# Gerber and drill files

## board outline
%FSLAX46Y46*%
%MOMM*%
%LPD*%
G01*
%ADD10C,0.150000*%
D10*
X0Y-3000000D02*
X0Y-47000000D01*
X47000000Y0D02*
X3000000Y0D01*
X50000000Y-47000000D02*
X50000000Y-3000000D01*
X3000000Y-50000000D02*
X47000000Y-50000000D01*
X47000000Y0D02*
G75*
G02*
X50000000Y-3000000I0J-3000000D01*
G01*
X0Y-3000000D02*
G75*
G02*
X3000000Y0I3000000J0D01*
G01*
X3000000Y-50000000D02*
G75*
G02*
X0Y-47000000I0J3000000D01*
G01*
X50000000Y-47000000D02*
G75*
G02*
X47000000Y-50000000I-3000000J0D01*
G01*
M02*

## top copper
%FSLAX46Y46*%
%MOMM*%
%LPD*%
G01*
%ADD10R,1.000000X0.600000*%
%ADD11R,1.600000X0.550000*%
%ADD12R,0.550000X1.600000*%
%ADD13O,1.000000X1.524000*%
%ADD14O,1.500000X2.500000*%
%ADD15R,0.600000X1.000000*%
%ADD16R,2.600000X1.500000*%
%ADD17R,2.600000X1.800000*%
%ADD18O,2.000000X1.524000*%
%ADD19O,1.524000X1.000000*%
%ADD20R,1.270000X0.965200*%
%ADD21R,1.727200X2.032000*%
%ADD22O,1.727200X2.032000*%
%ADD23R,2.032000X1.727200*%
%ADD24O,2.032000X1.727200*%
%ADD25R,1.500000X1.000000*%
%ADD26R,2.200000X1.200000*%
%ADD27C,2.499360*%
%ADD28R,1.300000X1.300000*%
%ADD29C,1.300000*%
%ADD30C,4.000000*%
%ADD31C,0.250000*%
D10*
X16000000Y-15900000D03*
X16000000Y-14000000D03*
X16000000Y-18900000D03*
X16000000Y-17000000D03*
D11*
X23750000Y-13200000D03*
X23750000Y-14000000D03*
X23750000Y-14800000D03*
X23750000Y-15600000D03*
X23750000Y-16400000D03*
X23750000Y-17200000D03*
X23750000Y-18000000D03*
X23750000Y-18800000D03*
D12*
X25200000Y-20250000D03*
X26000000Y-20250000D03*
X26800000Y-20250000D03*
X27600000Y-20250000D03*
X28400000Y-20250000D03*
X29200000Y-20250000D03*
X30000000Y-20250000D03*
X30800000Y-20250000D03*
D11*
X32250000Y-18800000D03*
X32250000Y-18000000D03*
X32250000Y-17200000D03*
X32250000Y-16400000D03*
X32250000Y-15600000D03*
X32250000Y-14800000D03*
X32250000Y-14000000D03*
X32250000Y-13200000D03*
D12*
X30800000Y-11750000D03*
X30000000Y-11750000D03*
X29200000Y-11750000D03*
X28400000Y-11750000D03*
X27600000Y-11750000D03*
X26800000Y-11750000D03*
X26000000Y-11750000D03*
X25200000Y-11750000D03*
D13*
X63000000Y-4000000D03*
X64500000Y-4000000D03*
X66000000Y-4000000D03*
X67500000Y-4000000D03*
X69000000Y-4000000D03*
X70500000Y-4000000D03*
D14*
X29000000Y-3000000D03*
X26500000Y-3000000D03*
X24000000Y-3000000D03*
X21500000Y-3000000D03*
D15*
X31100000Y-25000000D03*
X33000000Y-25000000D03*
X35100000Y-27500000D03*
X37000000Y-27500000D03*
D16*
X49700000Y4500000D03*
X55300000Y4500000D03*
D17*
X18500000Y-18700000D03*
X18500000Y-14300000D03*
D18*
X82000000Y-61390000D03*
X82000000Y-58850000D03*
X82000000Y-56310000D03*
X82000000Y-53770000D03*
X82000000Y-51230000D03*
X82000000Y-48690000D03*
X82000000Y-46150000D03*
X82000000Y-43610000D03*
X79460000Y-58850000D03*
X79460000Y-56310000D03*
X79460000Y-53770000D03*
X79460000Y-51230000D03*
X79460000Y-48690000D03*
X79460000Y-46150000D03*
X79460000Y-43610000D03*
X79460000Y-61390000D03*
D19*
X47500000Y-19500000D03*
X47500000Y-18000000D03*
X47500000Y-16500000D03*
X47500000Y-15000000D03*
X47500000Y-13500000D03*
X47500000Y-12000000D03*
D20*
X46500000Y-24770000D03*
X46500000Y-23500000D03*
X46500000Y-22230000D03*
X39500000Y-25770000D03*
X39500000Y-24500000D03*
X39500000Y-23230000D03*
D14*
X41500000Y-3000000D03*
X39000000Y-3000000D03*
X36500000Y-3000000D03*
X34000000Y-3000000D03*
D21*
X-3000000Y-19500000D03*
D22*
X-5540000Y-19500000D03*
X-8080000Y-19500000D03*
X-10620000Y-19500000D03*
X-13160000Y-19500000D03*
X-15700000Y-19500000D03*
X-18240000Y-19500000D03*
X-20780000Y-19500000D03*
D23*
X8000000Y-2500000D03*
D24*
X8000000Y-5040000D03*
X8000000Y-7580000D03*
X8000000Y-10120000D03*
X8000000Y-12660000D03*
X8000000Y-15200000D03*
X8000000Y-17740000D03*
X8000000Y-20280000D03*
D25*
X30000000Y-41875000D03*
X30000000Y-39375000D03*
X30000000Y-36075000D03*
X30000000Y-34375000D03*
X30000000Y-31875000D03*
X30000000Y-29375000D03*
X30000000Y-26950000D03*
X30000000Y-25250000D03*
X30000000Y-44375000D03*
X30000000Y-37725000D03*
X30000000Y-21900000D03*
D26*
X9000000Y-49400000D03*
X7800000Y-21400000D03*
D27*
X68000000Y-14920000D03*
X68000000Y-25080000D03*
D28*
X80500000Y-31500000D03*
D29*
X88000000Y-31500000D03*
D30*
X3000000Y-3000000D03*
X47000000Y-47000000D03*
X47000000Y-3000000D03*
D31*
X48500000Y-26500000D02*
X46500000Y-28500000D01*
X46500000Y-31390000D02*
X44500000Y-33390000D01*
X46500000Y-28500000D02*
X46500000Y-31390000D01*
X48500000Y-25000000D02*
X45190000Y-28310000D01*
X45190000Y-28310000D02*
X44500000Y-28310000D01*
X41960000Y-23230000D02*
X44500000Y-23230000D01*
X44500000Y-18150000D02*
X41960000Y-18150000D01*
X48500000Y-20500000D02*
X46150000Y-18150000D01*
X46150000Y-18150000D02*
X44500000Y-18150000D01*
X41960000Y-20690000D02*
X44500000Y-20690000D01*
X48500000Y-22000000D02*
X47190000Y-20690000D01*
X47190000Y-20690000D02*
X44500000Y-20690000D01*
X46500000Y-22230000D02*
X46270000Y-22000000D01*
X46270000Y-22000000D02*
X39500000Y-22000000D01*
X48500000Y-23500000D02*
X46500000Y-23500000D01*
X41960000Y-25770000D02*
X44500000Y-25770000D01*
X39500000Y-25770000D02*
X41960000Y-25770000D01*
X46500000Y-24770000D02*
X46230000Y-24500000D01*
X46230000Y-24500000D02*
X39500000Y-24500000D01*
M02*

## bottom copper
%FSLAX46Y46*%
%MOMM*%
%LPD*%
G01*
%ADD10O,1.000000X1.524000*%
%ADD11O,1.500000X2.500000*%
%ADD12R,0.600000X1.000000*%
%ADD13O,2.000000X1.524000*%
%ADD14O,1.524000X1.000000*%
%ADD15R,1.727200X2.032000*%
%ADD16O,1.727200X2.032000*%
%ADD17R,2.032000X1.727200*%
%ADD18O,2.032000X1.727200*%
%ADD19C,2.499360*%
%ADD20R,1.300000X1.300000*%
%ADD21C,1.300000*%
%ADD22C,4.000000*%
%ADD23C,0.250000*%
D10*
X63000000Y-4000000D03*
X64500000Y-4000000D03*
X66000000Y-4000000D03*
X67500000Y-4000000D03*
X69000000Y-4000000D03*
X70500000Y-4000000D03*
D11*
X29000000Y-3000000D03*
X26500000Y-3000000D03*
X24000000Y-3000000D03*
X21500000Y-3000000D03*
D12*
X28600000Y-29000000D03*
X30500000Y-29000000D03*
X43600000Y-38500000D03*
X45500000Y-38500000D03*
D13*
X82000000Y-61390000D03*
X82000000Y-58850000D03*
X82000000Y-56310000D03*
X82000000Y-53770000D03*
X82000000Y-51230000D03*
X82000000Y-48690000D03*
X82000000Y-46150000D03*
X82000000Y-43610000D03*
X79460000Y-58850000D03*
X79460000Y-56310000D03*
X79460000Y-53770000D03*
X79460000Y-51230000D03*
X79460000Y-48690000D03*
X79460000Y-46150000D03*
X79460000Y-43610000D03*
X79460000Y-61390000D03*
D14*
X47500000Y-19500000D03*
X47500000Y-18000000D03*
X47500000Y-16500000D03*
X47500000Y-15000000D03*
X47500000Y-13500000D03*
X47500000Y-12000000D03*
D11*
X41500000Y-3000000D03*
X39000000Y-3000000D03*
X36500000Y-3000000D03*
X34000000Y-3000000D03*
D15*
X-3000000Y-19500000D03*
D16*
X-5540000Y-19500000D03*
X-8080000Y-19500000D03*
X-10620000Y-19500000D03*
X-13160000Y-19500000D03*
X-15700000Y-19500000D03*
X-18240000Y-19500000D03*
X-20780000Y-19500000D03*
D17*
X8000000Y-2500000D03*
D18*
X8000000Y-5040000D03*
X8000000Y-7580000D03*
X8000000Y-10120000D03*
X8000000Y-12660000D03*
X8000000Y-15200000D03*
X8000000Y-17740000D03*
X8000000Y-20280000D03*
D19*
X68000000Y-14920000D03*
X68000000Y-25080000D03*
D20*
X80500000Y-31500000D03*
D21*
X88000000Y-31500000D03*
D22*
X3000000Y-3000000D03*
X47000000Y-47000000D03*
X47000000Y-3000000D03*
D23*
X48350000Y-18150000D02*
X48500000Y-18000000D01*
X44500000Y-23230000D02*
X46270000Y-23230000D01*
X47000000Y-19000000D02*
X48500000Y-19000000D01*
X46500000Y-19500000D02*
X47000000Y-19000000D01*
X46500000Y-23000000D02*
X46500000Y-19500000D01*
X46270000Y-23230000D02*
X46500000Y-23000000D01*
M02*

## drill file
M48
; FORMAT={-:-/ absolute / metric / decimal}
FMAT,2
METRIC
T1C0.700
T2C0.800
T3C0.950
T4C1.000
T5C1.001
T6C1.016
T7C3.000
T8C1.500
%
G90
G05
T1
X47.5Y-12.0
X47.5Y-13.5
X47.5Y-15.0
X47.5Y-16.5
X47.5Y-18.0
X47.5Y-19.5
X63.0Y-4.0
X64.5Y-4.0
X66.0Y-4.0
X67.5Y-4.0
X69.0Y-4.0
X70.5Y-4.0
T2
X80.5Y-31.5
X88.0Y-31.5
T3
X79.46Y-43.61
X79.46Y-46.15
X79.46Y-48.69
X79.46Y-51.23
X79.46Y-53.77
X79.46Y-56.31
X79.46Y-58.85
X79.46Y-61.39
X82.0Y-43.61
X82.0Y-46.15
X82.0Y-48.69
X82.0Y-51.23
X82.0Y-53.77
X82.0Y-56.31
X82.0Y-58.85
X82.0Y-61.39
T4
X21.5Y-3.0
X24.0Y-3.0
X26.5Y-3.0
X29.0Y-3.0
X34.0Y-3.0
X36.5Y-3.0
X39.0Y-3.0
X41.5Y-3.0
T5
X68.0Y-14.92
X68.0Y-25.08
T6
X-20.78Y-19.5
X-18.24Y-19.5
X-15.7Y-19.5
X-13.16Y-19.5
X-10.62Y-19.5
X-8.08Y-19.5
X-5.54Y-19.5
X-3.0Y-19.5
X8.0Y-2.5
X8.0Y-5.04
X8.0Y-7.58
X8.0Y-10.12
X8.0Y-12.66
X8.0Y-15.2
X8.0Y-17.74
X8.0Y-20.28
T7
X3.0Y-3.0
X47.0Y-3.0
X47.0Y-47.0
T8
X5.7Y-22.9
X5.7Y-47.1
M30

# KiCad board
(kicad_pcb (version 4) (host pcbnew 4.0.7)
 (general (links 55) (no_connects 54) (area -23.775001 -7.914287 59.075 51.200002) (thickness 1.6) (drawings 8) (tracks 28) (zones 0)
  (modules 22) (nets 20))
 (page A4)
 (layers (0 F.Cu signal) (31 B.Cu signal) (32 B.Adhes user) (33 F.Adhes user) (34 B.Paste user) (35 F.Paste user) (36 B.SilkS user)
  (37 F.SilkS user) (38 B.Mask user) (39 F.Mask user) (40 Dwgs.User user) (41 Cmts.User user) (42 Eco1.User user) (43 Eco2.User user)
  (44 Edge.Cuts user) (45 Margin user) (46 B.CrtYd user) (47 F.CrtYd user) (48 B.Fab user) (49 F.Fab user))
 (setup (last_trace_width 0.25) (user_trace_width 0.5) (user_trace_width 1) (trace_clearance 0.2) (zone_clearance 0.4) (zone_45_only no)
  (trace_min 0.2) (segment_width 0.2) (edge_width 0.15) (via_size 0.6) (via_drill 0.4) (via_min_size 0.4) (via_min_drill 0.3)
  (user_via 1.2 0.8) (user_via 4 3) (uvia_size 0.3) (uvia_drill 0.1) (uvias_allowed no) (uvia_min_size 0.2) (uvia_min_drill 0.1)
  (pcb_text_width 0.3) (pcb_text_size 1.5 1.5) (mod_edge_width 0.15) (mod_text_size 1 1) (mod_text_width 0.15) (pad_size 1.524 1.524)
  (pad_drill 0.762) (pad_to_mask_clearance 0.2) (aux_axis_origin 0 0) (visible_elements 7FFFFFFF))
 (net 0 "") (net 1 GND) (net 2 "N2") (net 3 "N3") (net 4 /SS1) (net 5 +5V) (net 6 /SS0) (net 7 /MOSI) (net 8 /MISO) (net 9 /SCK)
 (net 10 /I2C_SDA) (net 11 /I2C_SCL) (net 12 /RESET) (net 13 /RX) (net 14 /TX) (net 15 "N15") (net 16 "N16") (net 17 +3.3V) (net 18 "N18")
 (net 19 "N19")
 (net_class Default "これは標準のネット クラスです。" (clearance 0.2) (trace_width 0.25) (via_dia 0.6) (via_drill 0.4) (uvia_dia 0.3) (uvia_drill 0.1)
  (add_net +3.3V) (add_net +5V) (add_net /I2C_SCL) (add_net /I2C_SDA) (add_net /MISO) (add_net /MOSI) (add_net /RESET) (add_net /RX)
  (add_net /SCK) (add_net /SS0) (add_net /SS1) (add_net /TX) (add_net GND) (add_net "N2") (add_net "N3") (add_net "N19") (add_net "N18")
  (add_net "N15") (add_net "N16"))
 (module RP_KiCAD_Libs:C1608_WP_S (layer F.Cu) (at 16 15 90)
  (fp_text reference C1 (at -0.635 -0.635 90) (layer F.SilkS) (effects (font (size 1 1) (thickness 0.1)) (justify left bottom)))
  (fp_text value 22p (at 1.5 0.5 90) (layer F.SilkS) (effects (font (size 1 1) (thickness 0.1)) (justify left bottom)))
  (pad 1 smd rect (at -0.9 0 90) (size 0.6 1) (layers F.Cu F.Paste F.Mask) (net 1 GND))
  (pad 2 smd rect (at 1 0 90) (size 0.6 1) (layers F.Cu F.Paste F.Mask) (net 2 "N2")))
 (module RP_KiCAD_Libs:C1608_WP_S (layer F.Cu) (at 16 18 90)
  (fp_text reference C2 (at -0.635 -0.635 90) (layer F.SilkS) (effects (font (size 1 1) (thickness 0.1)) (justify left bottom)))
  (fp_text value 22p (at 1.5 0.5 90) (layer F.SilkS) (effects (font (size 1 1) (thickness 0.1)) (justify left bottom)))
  (pad 1 smd rect (at -0.9 0 90) (size 0.6 1) (layers F.Cu F.Paste F.Mask) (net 1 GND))
  (pad 2 smd rect (at 1 0 90) (size 0.6 1) (layers F.Cu F.Paste F.Mask) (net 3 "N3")))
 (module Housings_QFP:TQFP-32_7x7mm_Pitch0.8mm (layer F.Cu) (at 28 16)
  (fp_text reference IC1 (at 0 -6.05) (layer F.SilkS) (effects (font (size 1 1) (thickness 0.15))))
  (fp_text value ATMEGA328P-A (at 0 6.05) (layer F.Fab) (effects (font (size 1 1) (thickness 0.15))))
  (pad 1 smd rect (at -4.25 -2.8) (size 1.6 0.55) (layers F.Cu F.Paste F.Mask))
  (pad 2 smd rect (at -4.25 -2) (size 1.6 0.55) (layers F.Cu F.Paste F.Mask) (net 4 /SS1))
  (pad 3 smd rect (at -4.25 -1.2) (size 1.6 0.55) (layers F.Cu F.Paste F.Mask) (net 1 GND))
  (pad 4 smd rect (at -4.25 -0.4) (size 1.6 0.55) (layers F.Cu F.Paste F.Mask) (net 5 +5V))
  (pad 5 smd rect (at -4.25 0.4) (size 1.6 0.55) (layers F.Cu F.Paste F.Mask) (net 1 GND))
  (pad 6 smd rect (at -4.25 1.2) (size 1.6 0.55) (layers F.Cu F.Paste F.Mask) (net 5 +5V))
  (pad 7 smd rect (at -4.25 2) (size 1.6 0.55) (layers F.Cu F.Paste F.Mask) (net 2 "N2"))
  (pad 8 smd rect (at -4.25 2.8) (size 1.6 0.55) (layers F.Cu F.Paste F.Mask) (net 3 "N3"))
  (pad 9 smd rect (at -2.8 4.25 90) (size 1.6 0.55) (layers F.Cu F.Paste F.Mask))
  (pad 10 smd rect (at -2 4.25 90) (size 1.6 0.55) (layers F.Cu F.Paste F.Mask))
  (pad 11 smd rect (at -1.2 4.25 90) (size 1.6 0.55) (layers F.Cu F.Paste F.Mask))
  (pad 12 smd rect (at -0.4 4.25 90) (size 1.6 0.55) (layers F.Cu F.Paste F.Mask))
  (pad 13 smd rect (at 0.4 4.25 90) (size 1.6 0.55) (layers F.Cu F.Paste F.Mask))
  (pad 14 smd rect (at 1.2 4.25 90) (size 1.6 0.55) (layers F.Cu F.Paste F.Mask) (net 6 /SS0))
  (pad 15 smd rect (at 2 4.25 90) (size 1.6 0.55) (layers F.Cu F.Paste F.Mask) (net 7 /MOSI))
  (pad 16 smd rect (at 2.8 4.25 90) (size 1.6 0.55) (layers F.Cu F.Paste F.Mask) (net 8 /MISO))
  (pad 17 smd rect (at 4.25 2.8) (size 1.6 0.55) (layers F.Cu F.Paste F.Mask) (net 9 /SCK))
  (pad 18 smd rect (at 4.25 2) (size 1.6 0.55) (layers F.Cu F.Paste F.Mask) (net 5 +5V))
  (pad 19 smd rect (at 4.25 1.2) (size 1.6 0.55) (layers F.Cu F.Paste F.Mask))
  (pad 20 smd rect (at 4.25 0.4) (size 1.6 0.55) (layers F.Cu F.Paste F.Mask) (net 5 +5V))
  (pad 21 smd rect (at 4.25 -0.4) (size 1.6 0.55) (layers F.Cu F.Paste F.Mask) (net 1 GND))
  (pad 22 smd rect (at 4.25 -1.2) (size 1.6 0.55) (layers F.Cu F.Paste F.Mask))
  (pad 23 smd rect (at 4.25 -2) (size 1.6 0.55) (layers F.Cu F.Paste F.Mask))
  (pad 24 smd rect (at 4.25 -2.8) (size 1.6 0.55) (layers F.Cu F.Paste F.Mask))
  (pad 25 smd rect (at 2.8 -4.25 90) (size 1.6 0.55) (layers F.Cu F.Paste F.Mask))
  (pad 26 smd rect (at 2 -4.25 90) (size 1.6 0.55) (layers F.Cu F.Paste F.Mask))
  (pad 27 smd rect (at 1.2 -4.25 90) (size 1.6 0.55) (layers F.Cu F.Paste F.Mask) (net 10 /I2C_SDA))
  (pad 28 smd rect (at 0.4 -4.25 90) (size 1.6 0.55) (layers F.Cu F.Paste F.Mask) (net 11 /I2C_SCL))
  (pad 29 smd rect (at -0.4 -4.25 90) (size 1.6 0.55) (layers F.Cu F.Paste F.Mask) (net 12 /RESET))
  (pad 30 smd rect (at -1.2 -4.25 90) (size 1.6 0.55) (layers F.Cu F.Paste F.Mask) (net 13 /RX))
  (pad 31 smd rect (at -2 -4.25 90) (size 1.6 0.55) (layers F.Cu F.Paste F.Mask) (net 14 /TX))
  (pad 32 smd rect (at -2.8 -4.25 90) (size 1.6 0.55) (layers F.Cu F.Paste F.Mask)))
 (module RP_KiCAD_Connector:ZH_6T (layer F.Cu) (at 63 4)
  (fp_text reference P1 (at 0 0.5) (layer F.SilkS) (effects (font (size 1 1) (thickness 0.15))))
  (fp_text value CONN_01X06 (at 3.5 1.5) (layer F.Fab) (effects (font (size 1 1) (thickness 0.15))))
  (pad 1 thru_hole oval (at 0 0) (size 1 1.524) (drill 0.7) (layers *.Cu *.Mask) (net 1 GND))
  (pad 2 thru_hole oval (at 1.5 0) (size 1 1.524) (drill 0.7) (layers *.Cu *.Mask) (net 5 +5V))
  (pad 3 thru_hole oval (at 3 0) (size 1 1.524) (drill 0.7) (layers *.Cu *.Mask) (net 12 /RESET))
  (pad 4 thru_hole oval (at 4.5 0) (size 1 1.524) (drill 0.7) (layers *.Cu *.Mask))
  (pad 5 thru_hole oval (at 6 0) (size 1 1.524) (drill 0.7) (layers *.Cu *.Mask) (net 14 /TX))
  (pad 6 thru_hole oval (at 7.5 0) (size 1 1.524) (drill 0.7) (layers *.Cu *.Mask) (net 13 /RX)))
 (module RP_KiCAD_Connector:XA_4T (layer F.Cu) (at 29 3 180)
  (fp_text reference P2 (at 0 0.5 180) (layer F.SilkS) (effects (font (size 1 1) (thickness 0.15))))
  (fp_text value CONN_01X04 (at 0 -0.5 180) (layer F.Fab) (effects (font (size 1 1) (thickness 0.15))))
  (pad 4 thru_hole oval (at 0 0 180) (size 1.5 2.5) (drill 1) (layers *.Cu *.Mask F.SilkS) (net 14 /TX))
  (pad 3 thru_hole oval (at 2.5 0 180) (size 1.5 2.5) (drill 1) (layers *.Cu *.Mask F.SilkS) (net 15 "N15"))
  (pad 2 thru_hole oval (at 5 0 180) (size 1.5 2.5) (drill 1) (layers *.Cu *.Mask F.SilkS) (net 5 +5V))
  (pad 1 thru_hole oval (at 7.5 0 180) (size 1.5 2.5) (drill 1) (layers *.Cu *.Mask F.SilkS) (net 1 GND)))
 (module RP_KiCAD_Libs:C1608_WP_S (layer B.Cu) (at 29.5 29)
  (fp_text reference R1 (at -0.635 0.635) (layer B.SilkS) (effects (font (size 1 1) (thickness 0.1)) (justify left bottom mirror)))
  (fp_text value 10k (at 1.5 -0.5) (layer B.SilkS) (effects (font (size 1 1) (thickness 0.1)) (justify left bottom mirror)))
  (pad 1 smd rect (at -0.9 0) (size 0.6 1) (layers B.Cu B.Paste B.Mask))
  (pad 2 smd rect (at 1 0) (size 0.6 1) (layers B.Cu B.Paste B.Mask) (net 12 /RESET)))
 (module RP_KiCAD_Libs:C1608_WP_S (layer B.Cu) (at 44.5 38.5)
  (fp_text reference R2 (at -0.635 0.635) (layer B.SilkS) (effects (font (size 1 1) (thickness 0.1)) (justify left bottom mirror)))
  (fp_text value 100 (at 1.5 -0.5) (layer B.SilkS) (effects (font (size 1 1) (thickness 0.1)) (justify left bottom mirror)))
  (pad 1 smd rect (at -0.9 0) (size 0.6 1) (layers B.Cu B.Paste B.Mask) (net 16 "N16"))
  (pad 2 smd rect (at 1 0) (size 0.6 1) (layers B.Cu B.Paste B.Mask) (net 12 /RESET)))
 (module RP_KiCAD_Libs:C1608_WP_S (layer F.Cu) (at 32 25)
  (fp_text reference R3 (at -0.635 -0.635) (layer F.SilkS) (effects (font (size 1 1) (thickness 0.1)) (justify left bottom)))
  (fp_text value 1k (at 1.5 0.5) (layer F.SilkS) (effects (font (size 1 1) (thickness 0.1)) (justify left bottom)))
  (pad 1 smd rect (at -0.9 0) (size 0.6 1) (layers F.Cu F.Paste F.Mask) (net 14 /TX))
  (pad 2 smd rect (at 1 0) (size 0.6 1) (layers F.Cu F.Paste F.Mask)))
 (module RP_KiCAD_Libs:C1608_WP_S (layer F.Cu) (at 36 27.5)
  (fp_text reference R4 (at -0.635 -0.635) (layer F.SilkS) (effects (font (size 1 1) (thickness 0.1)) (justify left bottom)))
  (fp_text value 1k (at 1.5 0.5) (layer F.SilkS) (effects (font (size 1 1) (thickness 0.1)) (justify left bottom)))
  (pad 1 smd rect (at -0.9 0) (size 0.6 1) (layers F.Cu F.Paste F.Mask) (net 13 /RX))
  (pad 2 smd rect (at 1 0) (size 0.6 1) (layers F.Cu F.Paste F.Mask) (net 15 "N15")))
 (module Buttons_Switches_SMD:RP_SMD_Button (layer F.Cu) (at 52.5 -4.5 180)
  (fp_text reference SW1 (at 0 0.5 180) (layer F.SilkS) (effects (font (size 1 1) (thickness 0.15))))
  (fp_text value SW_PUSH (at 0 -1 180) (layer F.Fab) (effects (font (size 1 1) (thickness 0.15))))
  (pad 1 smd rect (at 2.8 0 180) (size 2.6 1.5) (layers F.Cu F.Paste F.Mask) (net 16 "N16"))
  (pad 2 smd rect (at -2.8 0 180) (size 2.6 1.5) (layers F.Cu F.Paste F.Mask) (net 1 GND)))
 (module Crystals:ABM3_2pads (layer F.Cu) (at 18.5 16.5 90)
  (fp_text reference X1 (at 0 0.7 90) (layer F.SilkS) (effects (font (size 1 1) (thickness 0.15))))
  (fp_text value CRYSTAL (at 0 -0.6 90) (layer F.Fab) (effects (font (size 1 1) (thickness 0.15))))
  (pad 1 smd rect (at -2.2 0 90) (size 1.8 2.6) (layers F.Cu F.Paste F.Mask) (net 3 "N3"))
  (pad 2 smd rect (at 2.2 0 90) (size 1.8 2.6) (layers F.Cu F.Paste F.Mask) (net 2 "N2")))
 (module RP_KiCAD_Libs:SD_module (layer B.Cu) (at 82 52.5)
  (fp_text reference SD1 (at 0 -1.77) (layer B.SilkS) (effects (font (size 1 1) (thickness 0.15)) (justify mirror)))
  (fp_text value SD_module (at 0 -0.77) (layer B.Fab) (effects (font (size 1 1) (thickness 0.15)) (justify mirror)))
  (pad 1 thru_hole oval (at 0 8.89) (size 2 1.524) (drill 0.95) (layers *.Cu *.Mask) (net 1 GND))
  (pad 2 thru_hole oval (at 0 6.35) (size 2 1.524) (drill 0.95) (layers *.Cu *.Mask) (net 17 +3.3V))
  (pad 3 thru_hole oval (at 0 3.81) (size 2 1.524) (drill 0.95) (layers *.Cu *.Mask) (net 5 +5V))
  (pad 4 thru_hole oval (at 0 1.27) (size 2 1.524) (drill 0.95) (layers *.Cu *.Mask) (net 6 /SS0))
  (pad 5 thru_hole oval (at 0 -1.27) (size 2 1.524) (drill 0.95) (layers *.Cu *.Mask) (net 7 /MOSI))
  (pad 6 thru_hole oval (at 0 -3.81) (size 2 1.524) (drill 0.95) (layers *.Cu *.Mask) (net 9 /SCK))
  (pad 7 thru_hole oval (at 0 -6.35) (size 2 1.524) (drill 0.95) (layers *.Cu *.Mask) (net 8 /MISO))
  (pad 8 thru_hole oval (at 0 -8.89) (size 2 1.524) (drill 0.95) (layers *.Cu *.Mask) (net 1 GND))
  (pad 2 thru_hole oval (at -2.54 6.35) (size 2 1.524) (drill 0.95) (layers *.Cu *.Mask) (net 17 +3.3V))
  (pad 3 thru_hole oval (at -2.54 3.81) (size 2 1.524) (drill 0.95) (layers *.Cu *.Mask) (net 5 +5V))
  (pad 4 thru_hole oval (at -2.54 1.27) (size 2 1.524) (drill 0.95) (layers *.Cu *.Mask) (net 6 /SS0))
  (pad 5 thru_hole oval (at -2.54 -1.27) (size 2 1.524) (drill 0.95) (layers *.Cu *.Mask) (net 7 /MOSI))
  (pad 6 thru_hole oval (at -2.54 -3.81) (size 2 1.524) (drill 0.95) (layers *.Cu *.Mask) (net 9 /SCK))
  (pad 7 thru_hole oval (at -2.54 -6.35) (size 2 1.524) (drill 0.95) (layers *.Cu *.Mask) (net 8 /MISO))
  (pad 8 thru_hole oval (at -2.54 -8.89) (size 2 1.524) (drill 0.95) (layers *.Cu *.Mask) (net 1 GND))
  (pad 1 thru_hole oval (at -2.54 8.89) (size 2 1.524) (drill 0.95) (layers *.Cu *.Mask) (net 1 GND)))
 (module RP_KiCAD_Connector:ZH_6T (layer F.Cu) (at 47.5 19.5 90)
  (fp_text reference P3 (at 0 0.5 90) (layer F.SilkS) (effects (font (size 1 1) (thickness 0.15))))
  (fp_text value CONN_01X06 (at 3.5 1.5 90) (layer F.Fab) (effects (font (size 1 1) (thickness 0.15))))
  (pad 1 thru_hole oval (at 0 0 90) (size 1 1.524) (drill 0.7) (layers *.Cu *.Mask) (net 1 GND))
  (pad 2 thru_hole oval (at 1.5 0 90) (size 1 1.524) (drill 0.7) (layers *.Cu *.Mask) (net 5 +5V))
  (pad 3 thru_hole oval (at 3 0 90) (size 1 1.524) (drill 0.7) (layers *.Cu *.Mask) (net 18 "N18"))
  (pad 4 thru_hole oval (at 4.5 0 90) (size 1 1.524) (drill 0.7) (layers *.Cu *.Mask) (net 9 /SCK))
  (pad 5 thru_hole oval (at 6 0 90) (size 1 1.524) (drill 0.7) (layers *.Cu *.Mask) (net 8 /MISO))
  (pad 6 thru_hole oval (at 7.5 0 90) (size 1 1.524) (drill 0.7) (layers *.Cu *.Mask) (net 7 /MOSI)))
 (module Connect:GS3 (layer F.Cu) (at 46.5 23.5 180)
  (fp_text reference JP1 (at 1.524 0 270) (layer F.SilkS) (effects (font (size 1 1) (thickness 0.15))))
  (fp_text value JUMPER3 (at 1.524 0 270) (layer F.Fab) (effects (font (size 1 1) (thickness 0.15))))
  (pad 1 smd rect (at 0 -1.27 180) (size 1.27 0.9652) (layers F.Cu F.Paste F.Mask) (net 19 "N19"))
  (pad 2 smd rect (at 0 0 180) (size 1.27 0.9652) (layers F.Cu F.Paste F.Mask) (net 18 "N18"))
  (pad 3 smd rect (at 0 1.27 180) (size 1.27 0.9652) (layers F.Cu F.Paste F.Mask) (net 12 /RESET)))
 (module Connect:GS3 (layer F.Cu) (at 39.5 24.5 180)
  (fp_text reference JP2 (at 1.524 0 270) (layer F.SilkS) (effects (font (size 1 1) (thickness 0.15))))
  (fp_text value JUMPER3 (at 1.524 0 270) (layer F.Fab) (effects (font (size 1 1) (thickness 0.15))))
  (pad 1 smd rect (at 0 -1.27 180) (size 1.27 0.9652) (layers F.Cu F.Paste F.Mask) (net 6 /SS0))
  (pad 2 smd rect (at 0 0 180) (size 1.27 0.9652) (layers F.Cu F.Paste F.Mask) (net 19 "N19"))
  (pad 3 smd rect (at 0 1.27 180) (size 1.27 0.9652) (layers F.Cu F.Paste F.Mask) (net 4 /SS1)))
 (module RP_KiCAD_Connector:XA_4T (layer F.Cu) (at 41.5 3 180)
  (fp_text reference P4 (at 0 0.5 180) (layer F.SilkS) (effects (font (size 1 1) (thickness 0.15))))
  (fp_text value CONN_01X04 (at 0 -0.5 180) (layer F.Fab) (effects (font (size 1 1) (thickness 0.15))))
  (pad 4 thru_hole oval (at 0 0 180) (size 1.5 2.5) (drill 1) (layers *.Cu *.Mask F.SilkS) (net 10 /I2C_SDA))
  (pad 3 thru_hole oval (at 2.5 0 180) (size 1.5 2.5) (drill 1) (layers *.Cu *.Mask F.SilkS) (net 11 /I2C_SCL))
  (pad 2 thru_hole oval (at 5 0 180) (size 1.5 2.5) (drill 1) (layers *.Cu *.Mask F.SilkS) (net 5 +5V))
  (pad 1 thru_hole oval (at 7.5 0 180) (size 1.5 2.5) (drill 1) (layers *.Cu *.Mask F.SilkS) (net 1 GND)))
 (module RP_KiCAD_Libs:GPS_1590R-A (layer F.Cu) (at -38.5 -13)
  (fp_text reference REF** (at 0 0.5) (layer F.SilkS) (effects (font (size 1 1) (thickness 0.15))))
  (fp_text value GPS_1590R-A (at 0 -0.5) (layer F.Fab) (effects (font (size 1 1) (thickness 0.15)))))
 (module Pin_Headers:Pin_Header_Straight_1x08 (layer F.Cu) (at -3 19.5 270)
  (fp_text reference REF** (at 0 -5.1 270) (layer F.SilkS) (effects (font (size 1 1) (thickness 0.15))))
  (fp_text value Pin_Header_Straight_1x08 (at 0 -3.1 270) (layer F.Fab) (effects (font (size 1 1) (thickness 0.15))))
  (pad 1 thru_hole rect (at 0 0 270) (size 2.032 1.7272) (drill 1.016) (layers *.Cu *.Mask F.SilkS))
  (pad 2 thru_hole oval (at 0 2.54 270) (size 2.032 1.7272) (drill 1.016) (layers *.Cu *.Mask F.SilkS))
  (pad 3 thru_hole oval (at 0 5.08 270) (size 2.032 1.7272) (drill 1.016) (layers *.Cu *.Mask F.SilkS))
  (pad 4 thru_hole oval (at 0 7.62 270) (size 2.032 1.7272) (drill 1.016) (layers *.Cu *.Mask F.SilkS))
  (pad 5 thru_hole oval (at 0 10.16 270) (size 2.032 1.7272) (drill 1.016) (layers *.Cu *.Mask F.SilkS))
  (pad 6 thru_hole oval (at 0 12.7 270) (size 2.032 1.7272) (drill 1.016) (layers *.Cu *.Mask F.SilkS))
  (pad 7 thru_hole oval (at 0 15.24 270) (size 2.032 1.7272) (drill 1.016) (layers *.Cu *.Mask F.SilkS))
  (pad 8 thru_hole oval (at 0 17.78 270) (size 2.032 1.7272) (drill 1.016) (layers *.Cu *.Mask F.SilkS)))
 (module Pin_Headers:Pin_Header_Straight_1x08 (layer F.Cu) (at 8 2.5)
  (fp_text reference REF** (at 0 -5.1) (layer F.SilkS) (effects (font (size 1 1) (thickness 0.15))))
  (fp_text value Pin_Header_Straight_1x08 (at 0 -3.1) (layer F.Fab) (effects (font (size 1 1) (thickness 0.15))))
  (pad 1 thru_hole rect (at 0 0) (size 2.032 1.7272) (drill 1.016) (layers *.Cu *.Mask F.SilkS))
  (pad 2 thru_hole oval (at 0 2.54) (size 2.032 1.7272) (drill 1.016) (layers *.Cu *.Mask F.SilkS))
  (pad 3 thru_hole oval (at 0 5.08) (size 2.032 1.7272) (drill 1.016) (layers *.Cu *.Mask F.SilkS))
  (pad 4 thru_hole oval (at 0 7.62) (size 2.032 1.7272) (drill 1.016) (layers *.Cu *.Mask F.SilkS))
  (pad 5 thru_hole oval (at 0 10.16) (size 2.032 1.7272) (drill 1.016) (layers *.Cu *.Mask F.SilkS))
  (pad 6 thru_hole oval (at 0 12.7) (size 2.032 1.7272) (drill 1.016) (layers *.Cu *.Mask F.SilkS))
  (pad 7 thru_hole oval (at 0 15.24) (size 2.032 1.7272) (drill 1.016) (layers *.Cu *.Mask F.SilkS))
  (pad 8 thru_hole oval (at 0 17.78) (size 2.032 1.7272) (drill 1.016) (layers *.Cu *.Mask F.SilkS)))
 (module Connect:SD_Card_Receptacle (layer F.Cu) (at 30 35 270)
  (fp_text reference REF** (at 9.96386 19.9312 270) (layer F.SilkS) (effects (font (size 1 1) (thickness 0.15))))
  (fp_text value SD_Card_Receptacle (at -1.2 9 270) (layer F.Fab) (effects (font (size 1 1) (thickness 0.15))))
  (pad 1 smd rect (at 6.875 0 270) (size 1 1.5) (layers F.Cu F.Paste F.Mask))
  (pad 2 smd rect (at 4.375 0 270) (size 1 1.5) (layers F.Cu F.Paste F.Mask))
  (pad 3 smd rect (at 1.075 0 270) (size 1 1.5) (layers F.Cu F.Paste F.Mask))
  (pad 4 smd rect (at -0.625 0 270) (size 1 1.5) (layers F.Cu F.Paste F.Mask))
  (pad 5 smd rect (at -3.125 0 270) (size 1 1.5) (layers F.Cu F.Paste F.Mask))
  (pad 6 smd rect (at -5.625 0 270) (size 1 1.5) (layers F.Cu F.Paste F.Mask))
  (pad 7 smd rect (at -8.05 0 270) (size 1 1.5) (layers F.Cu F.Paste F.Mask))
  (pad 8 smd rect (at -9.75 0 270) (size 1 1.5) (layers F.Cu F.Paste F.Mask))
  (pad 9 smd rect (at 9.375 0 270) (size 1 1.5) (layers F.Cu F.Paste F.Mask))
  (pad 10 smd rect (at 2.725 0 270) (size 1 1.5) (layers F.Cu F.Paste F.Mask))
  (pad 11 smd rect (at -13.1 0 270) (size 1 1.5) (layers F.Cu F.Paste F.Mask))
  (pad 12 smd rect (at 14.4 21 270) (size 1.2 2.2) (layers F.Cu F.Paste F.Mask))
  (pad 13 smd rect (at -13.6 22.2 270) (size 1.2 2.2) (layers F.Cu F.Paste F.Mask))
  (pad "" np_thru_hole circle (at 12.1 24.3 270) (size 1.5 1.5) (drill 1.5) (layers *.Cu *.Mask F.SilkS))
  (pad "" np_thru_hole circle (at -12.1 24.3 270) (size 1.5 1.5) (drill 1.5) (layers *.Cu *.Mask F.SilkS)))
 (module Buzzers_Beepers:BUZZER (layer F.Cu) (at 68 20 90)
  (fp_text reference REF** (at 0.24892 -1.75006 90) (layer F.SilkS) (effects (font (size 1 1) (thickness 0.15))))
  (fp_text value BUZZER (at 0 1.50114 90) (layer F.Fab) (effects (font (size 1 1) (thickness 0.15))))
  (pad 2 thru_hole circle (at 5.08 0 90) (size 2.49936 2.49936) (drill 1.00076) (layers *.Cu *.Mask F.SilkS))
  (pad 1 thru_hole circle (at -5.08 0 90) (size 2.49936 2.49936) (drill 1.00076) (layers *.Cu *.Mask F.SilkS)))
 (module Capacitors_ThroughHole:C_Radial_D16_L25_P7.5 (layer F.Cu) (at 80.5 31.5)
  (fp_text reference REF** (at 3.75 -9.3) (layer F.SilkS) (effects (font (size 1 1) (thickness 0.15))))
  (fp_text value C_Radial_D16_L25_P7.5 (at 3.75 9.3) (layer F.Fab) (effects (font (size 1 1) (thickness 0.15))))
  (pad 1 thru_hole rect (at 0 0) (size 1.3 1.3) (drill 0.8) (layers *.Cu *.Mask F.SilkS))
  (pad 2 thru_hole circle (at 7.5 0) (size 1.3 1.3) (drill 0.8) (layers *.Cu *.Mask F.SilkS)))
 (gr_line (start 0 3) (end 0 47) (angle 90) (layer Edge.Cuts) (width 0.15))
 (gr_line (start 47 0) (end 3 0) (angle 90) (layer Edge.Cuts) (width 0.15))
 (gr_line (start 50 47) (end 50 3) (angle 90) (layer Edge.Cuts) (width 0.15))
 (gr_line (start 3 50) (end 47 50) (angle 90) (layer Edge.Cuts) (width 0.15))
 (gr_arc (start 47 3) (end 47 0) (angle 90) (layer Edge.Cuts) (width 0.15))
 (gr_arc (start 3 3) (end 0 3) (angle 90) (layer Edge.Cuts) (width 0.15))
 (gr_arc (start 3 47) (end 3 50) (angle 90) (layer Edge.Cuts) (width 0.15))
 (gr_arc (start 47 47) (end 50 47) (angle 90) (layer Edge.Cuts) (width 0.15)) (via (at 3 3) (size 4) (drill 3) (layers F.Cu B.Cu) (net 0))
 (via (at 47 47) (size 4) (drill 3) (layers F.Cu B.Cu) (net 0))
 (via (at 47 3) (size 4) (drill 3) (layers F.Cu B.Cu) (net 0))
 (segment (start 48.35 18.15) (end 48.5 18) (width 0.25) (layer B.Cu) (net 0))
 (segment (start 48.5 26.5) (end 46.5 28.5) (width 0.25) (layer F.Cu) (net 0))
 (segment (start 46.5 31.39) (end 44.5 33.39) (width 0.25) (layer F.Cu) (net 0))
 (segment (start 46.5 28.5) (end 46.5 31.39) (width 0.25) (layer F.Cu) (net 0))
 (segment (start 48.5 25) (end 45.19 28.31) (width 0.25) (layer F.Cu) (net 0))
 (segment (start 45.19 28.31) (end 44.5 28.31) (width 0.25) (layer F.Cu) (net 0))
 (segment (start 44.5 23.23) (end 46.27 23.23) (width 0.25) (layer B.Cu) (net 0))
 (segment (start 47 19) (end 48.5 19) (width 0.25) (layer B.Cu) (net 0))
 (segment (start 46.5 19.5) (end 47 19) (width 0.25) (layer B.Cu) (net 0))
 (segment (start 46.5 23) (end 46.5 19.5) (width 0.25) (layer B.Cu) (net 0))
 (segment (start 46.27 23.23) (end 46.5 23) (width 0.25) (layer B.Cu) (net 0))
 (segment (start 41.96 23.23) (end 44.5 23.23) (width 0.25) (layer F.Cu) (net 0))
 (segment (start 44.5 18.15) (end 41.96 18.15) (width 0.25) (layer F.Cu) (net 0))
 (segment (start 48.5 20.5) (end 46.15 18.15) (width 0.25) (layer F.Cu) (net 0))
 (segment (start 46.15 18.15) (end 44.5 18.15) (width 0.25) (layer F.Cu) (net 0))
 (segment (start 41.96 20.69) (end 44.5 20.69) (width 0.25) (layer F.Cu) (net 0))
 (segment (start 48.5 22) (end 47.19 20.69) (width 0.25) (layer F.Cu) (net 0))
 (segment (start 47.19 20.69) (end 44.5 20.69) (width 0.25) (layer F.Cu) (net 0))
 (segment (start 46.5 22.23) (end 46.27 22) (width 0.25) (layer F.Cu) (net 12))
 (segment (start 46.27 22) (end 39.5 22) (width 0.25) (layer F.Cu) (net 12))
 (segment (start 48.5 23.5) (end 46.5 23.5) (width 0.25) (layer F.Cu) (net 18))
 (segment (start 41.96 25.77) (end 44.5 25.77) (width 0.25) (layer F.Cu) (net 6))
 (segment (start 39.5 25.77) (end 41.96 25.77) (width 0.25) (layer F.Cu) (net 6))
 (segment (start 46.5 24.77) (end 46.23 24.5) (width 0.25) (layer F.Cu) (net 19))
 (segment (start 46.23 24.5) (end 39.5 24.5) (width 0.25) (layer F.Cu) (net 19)))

